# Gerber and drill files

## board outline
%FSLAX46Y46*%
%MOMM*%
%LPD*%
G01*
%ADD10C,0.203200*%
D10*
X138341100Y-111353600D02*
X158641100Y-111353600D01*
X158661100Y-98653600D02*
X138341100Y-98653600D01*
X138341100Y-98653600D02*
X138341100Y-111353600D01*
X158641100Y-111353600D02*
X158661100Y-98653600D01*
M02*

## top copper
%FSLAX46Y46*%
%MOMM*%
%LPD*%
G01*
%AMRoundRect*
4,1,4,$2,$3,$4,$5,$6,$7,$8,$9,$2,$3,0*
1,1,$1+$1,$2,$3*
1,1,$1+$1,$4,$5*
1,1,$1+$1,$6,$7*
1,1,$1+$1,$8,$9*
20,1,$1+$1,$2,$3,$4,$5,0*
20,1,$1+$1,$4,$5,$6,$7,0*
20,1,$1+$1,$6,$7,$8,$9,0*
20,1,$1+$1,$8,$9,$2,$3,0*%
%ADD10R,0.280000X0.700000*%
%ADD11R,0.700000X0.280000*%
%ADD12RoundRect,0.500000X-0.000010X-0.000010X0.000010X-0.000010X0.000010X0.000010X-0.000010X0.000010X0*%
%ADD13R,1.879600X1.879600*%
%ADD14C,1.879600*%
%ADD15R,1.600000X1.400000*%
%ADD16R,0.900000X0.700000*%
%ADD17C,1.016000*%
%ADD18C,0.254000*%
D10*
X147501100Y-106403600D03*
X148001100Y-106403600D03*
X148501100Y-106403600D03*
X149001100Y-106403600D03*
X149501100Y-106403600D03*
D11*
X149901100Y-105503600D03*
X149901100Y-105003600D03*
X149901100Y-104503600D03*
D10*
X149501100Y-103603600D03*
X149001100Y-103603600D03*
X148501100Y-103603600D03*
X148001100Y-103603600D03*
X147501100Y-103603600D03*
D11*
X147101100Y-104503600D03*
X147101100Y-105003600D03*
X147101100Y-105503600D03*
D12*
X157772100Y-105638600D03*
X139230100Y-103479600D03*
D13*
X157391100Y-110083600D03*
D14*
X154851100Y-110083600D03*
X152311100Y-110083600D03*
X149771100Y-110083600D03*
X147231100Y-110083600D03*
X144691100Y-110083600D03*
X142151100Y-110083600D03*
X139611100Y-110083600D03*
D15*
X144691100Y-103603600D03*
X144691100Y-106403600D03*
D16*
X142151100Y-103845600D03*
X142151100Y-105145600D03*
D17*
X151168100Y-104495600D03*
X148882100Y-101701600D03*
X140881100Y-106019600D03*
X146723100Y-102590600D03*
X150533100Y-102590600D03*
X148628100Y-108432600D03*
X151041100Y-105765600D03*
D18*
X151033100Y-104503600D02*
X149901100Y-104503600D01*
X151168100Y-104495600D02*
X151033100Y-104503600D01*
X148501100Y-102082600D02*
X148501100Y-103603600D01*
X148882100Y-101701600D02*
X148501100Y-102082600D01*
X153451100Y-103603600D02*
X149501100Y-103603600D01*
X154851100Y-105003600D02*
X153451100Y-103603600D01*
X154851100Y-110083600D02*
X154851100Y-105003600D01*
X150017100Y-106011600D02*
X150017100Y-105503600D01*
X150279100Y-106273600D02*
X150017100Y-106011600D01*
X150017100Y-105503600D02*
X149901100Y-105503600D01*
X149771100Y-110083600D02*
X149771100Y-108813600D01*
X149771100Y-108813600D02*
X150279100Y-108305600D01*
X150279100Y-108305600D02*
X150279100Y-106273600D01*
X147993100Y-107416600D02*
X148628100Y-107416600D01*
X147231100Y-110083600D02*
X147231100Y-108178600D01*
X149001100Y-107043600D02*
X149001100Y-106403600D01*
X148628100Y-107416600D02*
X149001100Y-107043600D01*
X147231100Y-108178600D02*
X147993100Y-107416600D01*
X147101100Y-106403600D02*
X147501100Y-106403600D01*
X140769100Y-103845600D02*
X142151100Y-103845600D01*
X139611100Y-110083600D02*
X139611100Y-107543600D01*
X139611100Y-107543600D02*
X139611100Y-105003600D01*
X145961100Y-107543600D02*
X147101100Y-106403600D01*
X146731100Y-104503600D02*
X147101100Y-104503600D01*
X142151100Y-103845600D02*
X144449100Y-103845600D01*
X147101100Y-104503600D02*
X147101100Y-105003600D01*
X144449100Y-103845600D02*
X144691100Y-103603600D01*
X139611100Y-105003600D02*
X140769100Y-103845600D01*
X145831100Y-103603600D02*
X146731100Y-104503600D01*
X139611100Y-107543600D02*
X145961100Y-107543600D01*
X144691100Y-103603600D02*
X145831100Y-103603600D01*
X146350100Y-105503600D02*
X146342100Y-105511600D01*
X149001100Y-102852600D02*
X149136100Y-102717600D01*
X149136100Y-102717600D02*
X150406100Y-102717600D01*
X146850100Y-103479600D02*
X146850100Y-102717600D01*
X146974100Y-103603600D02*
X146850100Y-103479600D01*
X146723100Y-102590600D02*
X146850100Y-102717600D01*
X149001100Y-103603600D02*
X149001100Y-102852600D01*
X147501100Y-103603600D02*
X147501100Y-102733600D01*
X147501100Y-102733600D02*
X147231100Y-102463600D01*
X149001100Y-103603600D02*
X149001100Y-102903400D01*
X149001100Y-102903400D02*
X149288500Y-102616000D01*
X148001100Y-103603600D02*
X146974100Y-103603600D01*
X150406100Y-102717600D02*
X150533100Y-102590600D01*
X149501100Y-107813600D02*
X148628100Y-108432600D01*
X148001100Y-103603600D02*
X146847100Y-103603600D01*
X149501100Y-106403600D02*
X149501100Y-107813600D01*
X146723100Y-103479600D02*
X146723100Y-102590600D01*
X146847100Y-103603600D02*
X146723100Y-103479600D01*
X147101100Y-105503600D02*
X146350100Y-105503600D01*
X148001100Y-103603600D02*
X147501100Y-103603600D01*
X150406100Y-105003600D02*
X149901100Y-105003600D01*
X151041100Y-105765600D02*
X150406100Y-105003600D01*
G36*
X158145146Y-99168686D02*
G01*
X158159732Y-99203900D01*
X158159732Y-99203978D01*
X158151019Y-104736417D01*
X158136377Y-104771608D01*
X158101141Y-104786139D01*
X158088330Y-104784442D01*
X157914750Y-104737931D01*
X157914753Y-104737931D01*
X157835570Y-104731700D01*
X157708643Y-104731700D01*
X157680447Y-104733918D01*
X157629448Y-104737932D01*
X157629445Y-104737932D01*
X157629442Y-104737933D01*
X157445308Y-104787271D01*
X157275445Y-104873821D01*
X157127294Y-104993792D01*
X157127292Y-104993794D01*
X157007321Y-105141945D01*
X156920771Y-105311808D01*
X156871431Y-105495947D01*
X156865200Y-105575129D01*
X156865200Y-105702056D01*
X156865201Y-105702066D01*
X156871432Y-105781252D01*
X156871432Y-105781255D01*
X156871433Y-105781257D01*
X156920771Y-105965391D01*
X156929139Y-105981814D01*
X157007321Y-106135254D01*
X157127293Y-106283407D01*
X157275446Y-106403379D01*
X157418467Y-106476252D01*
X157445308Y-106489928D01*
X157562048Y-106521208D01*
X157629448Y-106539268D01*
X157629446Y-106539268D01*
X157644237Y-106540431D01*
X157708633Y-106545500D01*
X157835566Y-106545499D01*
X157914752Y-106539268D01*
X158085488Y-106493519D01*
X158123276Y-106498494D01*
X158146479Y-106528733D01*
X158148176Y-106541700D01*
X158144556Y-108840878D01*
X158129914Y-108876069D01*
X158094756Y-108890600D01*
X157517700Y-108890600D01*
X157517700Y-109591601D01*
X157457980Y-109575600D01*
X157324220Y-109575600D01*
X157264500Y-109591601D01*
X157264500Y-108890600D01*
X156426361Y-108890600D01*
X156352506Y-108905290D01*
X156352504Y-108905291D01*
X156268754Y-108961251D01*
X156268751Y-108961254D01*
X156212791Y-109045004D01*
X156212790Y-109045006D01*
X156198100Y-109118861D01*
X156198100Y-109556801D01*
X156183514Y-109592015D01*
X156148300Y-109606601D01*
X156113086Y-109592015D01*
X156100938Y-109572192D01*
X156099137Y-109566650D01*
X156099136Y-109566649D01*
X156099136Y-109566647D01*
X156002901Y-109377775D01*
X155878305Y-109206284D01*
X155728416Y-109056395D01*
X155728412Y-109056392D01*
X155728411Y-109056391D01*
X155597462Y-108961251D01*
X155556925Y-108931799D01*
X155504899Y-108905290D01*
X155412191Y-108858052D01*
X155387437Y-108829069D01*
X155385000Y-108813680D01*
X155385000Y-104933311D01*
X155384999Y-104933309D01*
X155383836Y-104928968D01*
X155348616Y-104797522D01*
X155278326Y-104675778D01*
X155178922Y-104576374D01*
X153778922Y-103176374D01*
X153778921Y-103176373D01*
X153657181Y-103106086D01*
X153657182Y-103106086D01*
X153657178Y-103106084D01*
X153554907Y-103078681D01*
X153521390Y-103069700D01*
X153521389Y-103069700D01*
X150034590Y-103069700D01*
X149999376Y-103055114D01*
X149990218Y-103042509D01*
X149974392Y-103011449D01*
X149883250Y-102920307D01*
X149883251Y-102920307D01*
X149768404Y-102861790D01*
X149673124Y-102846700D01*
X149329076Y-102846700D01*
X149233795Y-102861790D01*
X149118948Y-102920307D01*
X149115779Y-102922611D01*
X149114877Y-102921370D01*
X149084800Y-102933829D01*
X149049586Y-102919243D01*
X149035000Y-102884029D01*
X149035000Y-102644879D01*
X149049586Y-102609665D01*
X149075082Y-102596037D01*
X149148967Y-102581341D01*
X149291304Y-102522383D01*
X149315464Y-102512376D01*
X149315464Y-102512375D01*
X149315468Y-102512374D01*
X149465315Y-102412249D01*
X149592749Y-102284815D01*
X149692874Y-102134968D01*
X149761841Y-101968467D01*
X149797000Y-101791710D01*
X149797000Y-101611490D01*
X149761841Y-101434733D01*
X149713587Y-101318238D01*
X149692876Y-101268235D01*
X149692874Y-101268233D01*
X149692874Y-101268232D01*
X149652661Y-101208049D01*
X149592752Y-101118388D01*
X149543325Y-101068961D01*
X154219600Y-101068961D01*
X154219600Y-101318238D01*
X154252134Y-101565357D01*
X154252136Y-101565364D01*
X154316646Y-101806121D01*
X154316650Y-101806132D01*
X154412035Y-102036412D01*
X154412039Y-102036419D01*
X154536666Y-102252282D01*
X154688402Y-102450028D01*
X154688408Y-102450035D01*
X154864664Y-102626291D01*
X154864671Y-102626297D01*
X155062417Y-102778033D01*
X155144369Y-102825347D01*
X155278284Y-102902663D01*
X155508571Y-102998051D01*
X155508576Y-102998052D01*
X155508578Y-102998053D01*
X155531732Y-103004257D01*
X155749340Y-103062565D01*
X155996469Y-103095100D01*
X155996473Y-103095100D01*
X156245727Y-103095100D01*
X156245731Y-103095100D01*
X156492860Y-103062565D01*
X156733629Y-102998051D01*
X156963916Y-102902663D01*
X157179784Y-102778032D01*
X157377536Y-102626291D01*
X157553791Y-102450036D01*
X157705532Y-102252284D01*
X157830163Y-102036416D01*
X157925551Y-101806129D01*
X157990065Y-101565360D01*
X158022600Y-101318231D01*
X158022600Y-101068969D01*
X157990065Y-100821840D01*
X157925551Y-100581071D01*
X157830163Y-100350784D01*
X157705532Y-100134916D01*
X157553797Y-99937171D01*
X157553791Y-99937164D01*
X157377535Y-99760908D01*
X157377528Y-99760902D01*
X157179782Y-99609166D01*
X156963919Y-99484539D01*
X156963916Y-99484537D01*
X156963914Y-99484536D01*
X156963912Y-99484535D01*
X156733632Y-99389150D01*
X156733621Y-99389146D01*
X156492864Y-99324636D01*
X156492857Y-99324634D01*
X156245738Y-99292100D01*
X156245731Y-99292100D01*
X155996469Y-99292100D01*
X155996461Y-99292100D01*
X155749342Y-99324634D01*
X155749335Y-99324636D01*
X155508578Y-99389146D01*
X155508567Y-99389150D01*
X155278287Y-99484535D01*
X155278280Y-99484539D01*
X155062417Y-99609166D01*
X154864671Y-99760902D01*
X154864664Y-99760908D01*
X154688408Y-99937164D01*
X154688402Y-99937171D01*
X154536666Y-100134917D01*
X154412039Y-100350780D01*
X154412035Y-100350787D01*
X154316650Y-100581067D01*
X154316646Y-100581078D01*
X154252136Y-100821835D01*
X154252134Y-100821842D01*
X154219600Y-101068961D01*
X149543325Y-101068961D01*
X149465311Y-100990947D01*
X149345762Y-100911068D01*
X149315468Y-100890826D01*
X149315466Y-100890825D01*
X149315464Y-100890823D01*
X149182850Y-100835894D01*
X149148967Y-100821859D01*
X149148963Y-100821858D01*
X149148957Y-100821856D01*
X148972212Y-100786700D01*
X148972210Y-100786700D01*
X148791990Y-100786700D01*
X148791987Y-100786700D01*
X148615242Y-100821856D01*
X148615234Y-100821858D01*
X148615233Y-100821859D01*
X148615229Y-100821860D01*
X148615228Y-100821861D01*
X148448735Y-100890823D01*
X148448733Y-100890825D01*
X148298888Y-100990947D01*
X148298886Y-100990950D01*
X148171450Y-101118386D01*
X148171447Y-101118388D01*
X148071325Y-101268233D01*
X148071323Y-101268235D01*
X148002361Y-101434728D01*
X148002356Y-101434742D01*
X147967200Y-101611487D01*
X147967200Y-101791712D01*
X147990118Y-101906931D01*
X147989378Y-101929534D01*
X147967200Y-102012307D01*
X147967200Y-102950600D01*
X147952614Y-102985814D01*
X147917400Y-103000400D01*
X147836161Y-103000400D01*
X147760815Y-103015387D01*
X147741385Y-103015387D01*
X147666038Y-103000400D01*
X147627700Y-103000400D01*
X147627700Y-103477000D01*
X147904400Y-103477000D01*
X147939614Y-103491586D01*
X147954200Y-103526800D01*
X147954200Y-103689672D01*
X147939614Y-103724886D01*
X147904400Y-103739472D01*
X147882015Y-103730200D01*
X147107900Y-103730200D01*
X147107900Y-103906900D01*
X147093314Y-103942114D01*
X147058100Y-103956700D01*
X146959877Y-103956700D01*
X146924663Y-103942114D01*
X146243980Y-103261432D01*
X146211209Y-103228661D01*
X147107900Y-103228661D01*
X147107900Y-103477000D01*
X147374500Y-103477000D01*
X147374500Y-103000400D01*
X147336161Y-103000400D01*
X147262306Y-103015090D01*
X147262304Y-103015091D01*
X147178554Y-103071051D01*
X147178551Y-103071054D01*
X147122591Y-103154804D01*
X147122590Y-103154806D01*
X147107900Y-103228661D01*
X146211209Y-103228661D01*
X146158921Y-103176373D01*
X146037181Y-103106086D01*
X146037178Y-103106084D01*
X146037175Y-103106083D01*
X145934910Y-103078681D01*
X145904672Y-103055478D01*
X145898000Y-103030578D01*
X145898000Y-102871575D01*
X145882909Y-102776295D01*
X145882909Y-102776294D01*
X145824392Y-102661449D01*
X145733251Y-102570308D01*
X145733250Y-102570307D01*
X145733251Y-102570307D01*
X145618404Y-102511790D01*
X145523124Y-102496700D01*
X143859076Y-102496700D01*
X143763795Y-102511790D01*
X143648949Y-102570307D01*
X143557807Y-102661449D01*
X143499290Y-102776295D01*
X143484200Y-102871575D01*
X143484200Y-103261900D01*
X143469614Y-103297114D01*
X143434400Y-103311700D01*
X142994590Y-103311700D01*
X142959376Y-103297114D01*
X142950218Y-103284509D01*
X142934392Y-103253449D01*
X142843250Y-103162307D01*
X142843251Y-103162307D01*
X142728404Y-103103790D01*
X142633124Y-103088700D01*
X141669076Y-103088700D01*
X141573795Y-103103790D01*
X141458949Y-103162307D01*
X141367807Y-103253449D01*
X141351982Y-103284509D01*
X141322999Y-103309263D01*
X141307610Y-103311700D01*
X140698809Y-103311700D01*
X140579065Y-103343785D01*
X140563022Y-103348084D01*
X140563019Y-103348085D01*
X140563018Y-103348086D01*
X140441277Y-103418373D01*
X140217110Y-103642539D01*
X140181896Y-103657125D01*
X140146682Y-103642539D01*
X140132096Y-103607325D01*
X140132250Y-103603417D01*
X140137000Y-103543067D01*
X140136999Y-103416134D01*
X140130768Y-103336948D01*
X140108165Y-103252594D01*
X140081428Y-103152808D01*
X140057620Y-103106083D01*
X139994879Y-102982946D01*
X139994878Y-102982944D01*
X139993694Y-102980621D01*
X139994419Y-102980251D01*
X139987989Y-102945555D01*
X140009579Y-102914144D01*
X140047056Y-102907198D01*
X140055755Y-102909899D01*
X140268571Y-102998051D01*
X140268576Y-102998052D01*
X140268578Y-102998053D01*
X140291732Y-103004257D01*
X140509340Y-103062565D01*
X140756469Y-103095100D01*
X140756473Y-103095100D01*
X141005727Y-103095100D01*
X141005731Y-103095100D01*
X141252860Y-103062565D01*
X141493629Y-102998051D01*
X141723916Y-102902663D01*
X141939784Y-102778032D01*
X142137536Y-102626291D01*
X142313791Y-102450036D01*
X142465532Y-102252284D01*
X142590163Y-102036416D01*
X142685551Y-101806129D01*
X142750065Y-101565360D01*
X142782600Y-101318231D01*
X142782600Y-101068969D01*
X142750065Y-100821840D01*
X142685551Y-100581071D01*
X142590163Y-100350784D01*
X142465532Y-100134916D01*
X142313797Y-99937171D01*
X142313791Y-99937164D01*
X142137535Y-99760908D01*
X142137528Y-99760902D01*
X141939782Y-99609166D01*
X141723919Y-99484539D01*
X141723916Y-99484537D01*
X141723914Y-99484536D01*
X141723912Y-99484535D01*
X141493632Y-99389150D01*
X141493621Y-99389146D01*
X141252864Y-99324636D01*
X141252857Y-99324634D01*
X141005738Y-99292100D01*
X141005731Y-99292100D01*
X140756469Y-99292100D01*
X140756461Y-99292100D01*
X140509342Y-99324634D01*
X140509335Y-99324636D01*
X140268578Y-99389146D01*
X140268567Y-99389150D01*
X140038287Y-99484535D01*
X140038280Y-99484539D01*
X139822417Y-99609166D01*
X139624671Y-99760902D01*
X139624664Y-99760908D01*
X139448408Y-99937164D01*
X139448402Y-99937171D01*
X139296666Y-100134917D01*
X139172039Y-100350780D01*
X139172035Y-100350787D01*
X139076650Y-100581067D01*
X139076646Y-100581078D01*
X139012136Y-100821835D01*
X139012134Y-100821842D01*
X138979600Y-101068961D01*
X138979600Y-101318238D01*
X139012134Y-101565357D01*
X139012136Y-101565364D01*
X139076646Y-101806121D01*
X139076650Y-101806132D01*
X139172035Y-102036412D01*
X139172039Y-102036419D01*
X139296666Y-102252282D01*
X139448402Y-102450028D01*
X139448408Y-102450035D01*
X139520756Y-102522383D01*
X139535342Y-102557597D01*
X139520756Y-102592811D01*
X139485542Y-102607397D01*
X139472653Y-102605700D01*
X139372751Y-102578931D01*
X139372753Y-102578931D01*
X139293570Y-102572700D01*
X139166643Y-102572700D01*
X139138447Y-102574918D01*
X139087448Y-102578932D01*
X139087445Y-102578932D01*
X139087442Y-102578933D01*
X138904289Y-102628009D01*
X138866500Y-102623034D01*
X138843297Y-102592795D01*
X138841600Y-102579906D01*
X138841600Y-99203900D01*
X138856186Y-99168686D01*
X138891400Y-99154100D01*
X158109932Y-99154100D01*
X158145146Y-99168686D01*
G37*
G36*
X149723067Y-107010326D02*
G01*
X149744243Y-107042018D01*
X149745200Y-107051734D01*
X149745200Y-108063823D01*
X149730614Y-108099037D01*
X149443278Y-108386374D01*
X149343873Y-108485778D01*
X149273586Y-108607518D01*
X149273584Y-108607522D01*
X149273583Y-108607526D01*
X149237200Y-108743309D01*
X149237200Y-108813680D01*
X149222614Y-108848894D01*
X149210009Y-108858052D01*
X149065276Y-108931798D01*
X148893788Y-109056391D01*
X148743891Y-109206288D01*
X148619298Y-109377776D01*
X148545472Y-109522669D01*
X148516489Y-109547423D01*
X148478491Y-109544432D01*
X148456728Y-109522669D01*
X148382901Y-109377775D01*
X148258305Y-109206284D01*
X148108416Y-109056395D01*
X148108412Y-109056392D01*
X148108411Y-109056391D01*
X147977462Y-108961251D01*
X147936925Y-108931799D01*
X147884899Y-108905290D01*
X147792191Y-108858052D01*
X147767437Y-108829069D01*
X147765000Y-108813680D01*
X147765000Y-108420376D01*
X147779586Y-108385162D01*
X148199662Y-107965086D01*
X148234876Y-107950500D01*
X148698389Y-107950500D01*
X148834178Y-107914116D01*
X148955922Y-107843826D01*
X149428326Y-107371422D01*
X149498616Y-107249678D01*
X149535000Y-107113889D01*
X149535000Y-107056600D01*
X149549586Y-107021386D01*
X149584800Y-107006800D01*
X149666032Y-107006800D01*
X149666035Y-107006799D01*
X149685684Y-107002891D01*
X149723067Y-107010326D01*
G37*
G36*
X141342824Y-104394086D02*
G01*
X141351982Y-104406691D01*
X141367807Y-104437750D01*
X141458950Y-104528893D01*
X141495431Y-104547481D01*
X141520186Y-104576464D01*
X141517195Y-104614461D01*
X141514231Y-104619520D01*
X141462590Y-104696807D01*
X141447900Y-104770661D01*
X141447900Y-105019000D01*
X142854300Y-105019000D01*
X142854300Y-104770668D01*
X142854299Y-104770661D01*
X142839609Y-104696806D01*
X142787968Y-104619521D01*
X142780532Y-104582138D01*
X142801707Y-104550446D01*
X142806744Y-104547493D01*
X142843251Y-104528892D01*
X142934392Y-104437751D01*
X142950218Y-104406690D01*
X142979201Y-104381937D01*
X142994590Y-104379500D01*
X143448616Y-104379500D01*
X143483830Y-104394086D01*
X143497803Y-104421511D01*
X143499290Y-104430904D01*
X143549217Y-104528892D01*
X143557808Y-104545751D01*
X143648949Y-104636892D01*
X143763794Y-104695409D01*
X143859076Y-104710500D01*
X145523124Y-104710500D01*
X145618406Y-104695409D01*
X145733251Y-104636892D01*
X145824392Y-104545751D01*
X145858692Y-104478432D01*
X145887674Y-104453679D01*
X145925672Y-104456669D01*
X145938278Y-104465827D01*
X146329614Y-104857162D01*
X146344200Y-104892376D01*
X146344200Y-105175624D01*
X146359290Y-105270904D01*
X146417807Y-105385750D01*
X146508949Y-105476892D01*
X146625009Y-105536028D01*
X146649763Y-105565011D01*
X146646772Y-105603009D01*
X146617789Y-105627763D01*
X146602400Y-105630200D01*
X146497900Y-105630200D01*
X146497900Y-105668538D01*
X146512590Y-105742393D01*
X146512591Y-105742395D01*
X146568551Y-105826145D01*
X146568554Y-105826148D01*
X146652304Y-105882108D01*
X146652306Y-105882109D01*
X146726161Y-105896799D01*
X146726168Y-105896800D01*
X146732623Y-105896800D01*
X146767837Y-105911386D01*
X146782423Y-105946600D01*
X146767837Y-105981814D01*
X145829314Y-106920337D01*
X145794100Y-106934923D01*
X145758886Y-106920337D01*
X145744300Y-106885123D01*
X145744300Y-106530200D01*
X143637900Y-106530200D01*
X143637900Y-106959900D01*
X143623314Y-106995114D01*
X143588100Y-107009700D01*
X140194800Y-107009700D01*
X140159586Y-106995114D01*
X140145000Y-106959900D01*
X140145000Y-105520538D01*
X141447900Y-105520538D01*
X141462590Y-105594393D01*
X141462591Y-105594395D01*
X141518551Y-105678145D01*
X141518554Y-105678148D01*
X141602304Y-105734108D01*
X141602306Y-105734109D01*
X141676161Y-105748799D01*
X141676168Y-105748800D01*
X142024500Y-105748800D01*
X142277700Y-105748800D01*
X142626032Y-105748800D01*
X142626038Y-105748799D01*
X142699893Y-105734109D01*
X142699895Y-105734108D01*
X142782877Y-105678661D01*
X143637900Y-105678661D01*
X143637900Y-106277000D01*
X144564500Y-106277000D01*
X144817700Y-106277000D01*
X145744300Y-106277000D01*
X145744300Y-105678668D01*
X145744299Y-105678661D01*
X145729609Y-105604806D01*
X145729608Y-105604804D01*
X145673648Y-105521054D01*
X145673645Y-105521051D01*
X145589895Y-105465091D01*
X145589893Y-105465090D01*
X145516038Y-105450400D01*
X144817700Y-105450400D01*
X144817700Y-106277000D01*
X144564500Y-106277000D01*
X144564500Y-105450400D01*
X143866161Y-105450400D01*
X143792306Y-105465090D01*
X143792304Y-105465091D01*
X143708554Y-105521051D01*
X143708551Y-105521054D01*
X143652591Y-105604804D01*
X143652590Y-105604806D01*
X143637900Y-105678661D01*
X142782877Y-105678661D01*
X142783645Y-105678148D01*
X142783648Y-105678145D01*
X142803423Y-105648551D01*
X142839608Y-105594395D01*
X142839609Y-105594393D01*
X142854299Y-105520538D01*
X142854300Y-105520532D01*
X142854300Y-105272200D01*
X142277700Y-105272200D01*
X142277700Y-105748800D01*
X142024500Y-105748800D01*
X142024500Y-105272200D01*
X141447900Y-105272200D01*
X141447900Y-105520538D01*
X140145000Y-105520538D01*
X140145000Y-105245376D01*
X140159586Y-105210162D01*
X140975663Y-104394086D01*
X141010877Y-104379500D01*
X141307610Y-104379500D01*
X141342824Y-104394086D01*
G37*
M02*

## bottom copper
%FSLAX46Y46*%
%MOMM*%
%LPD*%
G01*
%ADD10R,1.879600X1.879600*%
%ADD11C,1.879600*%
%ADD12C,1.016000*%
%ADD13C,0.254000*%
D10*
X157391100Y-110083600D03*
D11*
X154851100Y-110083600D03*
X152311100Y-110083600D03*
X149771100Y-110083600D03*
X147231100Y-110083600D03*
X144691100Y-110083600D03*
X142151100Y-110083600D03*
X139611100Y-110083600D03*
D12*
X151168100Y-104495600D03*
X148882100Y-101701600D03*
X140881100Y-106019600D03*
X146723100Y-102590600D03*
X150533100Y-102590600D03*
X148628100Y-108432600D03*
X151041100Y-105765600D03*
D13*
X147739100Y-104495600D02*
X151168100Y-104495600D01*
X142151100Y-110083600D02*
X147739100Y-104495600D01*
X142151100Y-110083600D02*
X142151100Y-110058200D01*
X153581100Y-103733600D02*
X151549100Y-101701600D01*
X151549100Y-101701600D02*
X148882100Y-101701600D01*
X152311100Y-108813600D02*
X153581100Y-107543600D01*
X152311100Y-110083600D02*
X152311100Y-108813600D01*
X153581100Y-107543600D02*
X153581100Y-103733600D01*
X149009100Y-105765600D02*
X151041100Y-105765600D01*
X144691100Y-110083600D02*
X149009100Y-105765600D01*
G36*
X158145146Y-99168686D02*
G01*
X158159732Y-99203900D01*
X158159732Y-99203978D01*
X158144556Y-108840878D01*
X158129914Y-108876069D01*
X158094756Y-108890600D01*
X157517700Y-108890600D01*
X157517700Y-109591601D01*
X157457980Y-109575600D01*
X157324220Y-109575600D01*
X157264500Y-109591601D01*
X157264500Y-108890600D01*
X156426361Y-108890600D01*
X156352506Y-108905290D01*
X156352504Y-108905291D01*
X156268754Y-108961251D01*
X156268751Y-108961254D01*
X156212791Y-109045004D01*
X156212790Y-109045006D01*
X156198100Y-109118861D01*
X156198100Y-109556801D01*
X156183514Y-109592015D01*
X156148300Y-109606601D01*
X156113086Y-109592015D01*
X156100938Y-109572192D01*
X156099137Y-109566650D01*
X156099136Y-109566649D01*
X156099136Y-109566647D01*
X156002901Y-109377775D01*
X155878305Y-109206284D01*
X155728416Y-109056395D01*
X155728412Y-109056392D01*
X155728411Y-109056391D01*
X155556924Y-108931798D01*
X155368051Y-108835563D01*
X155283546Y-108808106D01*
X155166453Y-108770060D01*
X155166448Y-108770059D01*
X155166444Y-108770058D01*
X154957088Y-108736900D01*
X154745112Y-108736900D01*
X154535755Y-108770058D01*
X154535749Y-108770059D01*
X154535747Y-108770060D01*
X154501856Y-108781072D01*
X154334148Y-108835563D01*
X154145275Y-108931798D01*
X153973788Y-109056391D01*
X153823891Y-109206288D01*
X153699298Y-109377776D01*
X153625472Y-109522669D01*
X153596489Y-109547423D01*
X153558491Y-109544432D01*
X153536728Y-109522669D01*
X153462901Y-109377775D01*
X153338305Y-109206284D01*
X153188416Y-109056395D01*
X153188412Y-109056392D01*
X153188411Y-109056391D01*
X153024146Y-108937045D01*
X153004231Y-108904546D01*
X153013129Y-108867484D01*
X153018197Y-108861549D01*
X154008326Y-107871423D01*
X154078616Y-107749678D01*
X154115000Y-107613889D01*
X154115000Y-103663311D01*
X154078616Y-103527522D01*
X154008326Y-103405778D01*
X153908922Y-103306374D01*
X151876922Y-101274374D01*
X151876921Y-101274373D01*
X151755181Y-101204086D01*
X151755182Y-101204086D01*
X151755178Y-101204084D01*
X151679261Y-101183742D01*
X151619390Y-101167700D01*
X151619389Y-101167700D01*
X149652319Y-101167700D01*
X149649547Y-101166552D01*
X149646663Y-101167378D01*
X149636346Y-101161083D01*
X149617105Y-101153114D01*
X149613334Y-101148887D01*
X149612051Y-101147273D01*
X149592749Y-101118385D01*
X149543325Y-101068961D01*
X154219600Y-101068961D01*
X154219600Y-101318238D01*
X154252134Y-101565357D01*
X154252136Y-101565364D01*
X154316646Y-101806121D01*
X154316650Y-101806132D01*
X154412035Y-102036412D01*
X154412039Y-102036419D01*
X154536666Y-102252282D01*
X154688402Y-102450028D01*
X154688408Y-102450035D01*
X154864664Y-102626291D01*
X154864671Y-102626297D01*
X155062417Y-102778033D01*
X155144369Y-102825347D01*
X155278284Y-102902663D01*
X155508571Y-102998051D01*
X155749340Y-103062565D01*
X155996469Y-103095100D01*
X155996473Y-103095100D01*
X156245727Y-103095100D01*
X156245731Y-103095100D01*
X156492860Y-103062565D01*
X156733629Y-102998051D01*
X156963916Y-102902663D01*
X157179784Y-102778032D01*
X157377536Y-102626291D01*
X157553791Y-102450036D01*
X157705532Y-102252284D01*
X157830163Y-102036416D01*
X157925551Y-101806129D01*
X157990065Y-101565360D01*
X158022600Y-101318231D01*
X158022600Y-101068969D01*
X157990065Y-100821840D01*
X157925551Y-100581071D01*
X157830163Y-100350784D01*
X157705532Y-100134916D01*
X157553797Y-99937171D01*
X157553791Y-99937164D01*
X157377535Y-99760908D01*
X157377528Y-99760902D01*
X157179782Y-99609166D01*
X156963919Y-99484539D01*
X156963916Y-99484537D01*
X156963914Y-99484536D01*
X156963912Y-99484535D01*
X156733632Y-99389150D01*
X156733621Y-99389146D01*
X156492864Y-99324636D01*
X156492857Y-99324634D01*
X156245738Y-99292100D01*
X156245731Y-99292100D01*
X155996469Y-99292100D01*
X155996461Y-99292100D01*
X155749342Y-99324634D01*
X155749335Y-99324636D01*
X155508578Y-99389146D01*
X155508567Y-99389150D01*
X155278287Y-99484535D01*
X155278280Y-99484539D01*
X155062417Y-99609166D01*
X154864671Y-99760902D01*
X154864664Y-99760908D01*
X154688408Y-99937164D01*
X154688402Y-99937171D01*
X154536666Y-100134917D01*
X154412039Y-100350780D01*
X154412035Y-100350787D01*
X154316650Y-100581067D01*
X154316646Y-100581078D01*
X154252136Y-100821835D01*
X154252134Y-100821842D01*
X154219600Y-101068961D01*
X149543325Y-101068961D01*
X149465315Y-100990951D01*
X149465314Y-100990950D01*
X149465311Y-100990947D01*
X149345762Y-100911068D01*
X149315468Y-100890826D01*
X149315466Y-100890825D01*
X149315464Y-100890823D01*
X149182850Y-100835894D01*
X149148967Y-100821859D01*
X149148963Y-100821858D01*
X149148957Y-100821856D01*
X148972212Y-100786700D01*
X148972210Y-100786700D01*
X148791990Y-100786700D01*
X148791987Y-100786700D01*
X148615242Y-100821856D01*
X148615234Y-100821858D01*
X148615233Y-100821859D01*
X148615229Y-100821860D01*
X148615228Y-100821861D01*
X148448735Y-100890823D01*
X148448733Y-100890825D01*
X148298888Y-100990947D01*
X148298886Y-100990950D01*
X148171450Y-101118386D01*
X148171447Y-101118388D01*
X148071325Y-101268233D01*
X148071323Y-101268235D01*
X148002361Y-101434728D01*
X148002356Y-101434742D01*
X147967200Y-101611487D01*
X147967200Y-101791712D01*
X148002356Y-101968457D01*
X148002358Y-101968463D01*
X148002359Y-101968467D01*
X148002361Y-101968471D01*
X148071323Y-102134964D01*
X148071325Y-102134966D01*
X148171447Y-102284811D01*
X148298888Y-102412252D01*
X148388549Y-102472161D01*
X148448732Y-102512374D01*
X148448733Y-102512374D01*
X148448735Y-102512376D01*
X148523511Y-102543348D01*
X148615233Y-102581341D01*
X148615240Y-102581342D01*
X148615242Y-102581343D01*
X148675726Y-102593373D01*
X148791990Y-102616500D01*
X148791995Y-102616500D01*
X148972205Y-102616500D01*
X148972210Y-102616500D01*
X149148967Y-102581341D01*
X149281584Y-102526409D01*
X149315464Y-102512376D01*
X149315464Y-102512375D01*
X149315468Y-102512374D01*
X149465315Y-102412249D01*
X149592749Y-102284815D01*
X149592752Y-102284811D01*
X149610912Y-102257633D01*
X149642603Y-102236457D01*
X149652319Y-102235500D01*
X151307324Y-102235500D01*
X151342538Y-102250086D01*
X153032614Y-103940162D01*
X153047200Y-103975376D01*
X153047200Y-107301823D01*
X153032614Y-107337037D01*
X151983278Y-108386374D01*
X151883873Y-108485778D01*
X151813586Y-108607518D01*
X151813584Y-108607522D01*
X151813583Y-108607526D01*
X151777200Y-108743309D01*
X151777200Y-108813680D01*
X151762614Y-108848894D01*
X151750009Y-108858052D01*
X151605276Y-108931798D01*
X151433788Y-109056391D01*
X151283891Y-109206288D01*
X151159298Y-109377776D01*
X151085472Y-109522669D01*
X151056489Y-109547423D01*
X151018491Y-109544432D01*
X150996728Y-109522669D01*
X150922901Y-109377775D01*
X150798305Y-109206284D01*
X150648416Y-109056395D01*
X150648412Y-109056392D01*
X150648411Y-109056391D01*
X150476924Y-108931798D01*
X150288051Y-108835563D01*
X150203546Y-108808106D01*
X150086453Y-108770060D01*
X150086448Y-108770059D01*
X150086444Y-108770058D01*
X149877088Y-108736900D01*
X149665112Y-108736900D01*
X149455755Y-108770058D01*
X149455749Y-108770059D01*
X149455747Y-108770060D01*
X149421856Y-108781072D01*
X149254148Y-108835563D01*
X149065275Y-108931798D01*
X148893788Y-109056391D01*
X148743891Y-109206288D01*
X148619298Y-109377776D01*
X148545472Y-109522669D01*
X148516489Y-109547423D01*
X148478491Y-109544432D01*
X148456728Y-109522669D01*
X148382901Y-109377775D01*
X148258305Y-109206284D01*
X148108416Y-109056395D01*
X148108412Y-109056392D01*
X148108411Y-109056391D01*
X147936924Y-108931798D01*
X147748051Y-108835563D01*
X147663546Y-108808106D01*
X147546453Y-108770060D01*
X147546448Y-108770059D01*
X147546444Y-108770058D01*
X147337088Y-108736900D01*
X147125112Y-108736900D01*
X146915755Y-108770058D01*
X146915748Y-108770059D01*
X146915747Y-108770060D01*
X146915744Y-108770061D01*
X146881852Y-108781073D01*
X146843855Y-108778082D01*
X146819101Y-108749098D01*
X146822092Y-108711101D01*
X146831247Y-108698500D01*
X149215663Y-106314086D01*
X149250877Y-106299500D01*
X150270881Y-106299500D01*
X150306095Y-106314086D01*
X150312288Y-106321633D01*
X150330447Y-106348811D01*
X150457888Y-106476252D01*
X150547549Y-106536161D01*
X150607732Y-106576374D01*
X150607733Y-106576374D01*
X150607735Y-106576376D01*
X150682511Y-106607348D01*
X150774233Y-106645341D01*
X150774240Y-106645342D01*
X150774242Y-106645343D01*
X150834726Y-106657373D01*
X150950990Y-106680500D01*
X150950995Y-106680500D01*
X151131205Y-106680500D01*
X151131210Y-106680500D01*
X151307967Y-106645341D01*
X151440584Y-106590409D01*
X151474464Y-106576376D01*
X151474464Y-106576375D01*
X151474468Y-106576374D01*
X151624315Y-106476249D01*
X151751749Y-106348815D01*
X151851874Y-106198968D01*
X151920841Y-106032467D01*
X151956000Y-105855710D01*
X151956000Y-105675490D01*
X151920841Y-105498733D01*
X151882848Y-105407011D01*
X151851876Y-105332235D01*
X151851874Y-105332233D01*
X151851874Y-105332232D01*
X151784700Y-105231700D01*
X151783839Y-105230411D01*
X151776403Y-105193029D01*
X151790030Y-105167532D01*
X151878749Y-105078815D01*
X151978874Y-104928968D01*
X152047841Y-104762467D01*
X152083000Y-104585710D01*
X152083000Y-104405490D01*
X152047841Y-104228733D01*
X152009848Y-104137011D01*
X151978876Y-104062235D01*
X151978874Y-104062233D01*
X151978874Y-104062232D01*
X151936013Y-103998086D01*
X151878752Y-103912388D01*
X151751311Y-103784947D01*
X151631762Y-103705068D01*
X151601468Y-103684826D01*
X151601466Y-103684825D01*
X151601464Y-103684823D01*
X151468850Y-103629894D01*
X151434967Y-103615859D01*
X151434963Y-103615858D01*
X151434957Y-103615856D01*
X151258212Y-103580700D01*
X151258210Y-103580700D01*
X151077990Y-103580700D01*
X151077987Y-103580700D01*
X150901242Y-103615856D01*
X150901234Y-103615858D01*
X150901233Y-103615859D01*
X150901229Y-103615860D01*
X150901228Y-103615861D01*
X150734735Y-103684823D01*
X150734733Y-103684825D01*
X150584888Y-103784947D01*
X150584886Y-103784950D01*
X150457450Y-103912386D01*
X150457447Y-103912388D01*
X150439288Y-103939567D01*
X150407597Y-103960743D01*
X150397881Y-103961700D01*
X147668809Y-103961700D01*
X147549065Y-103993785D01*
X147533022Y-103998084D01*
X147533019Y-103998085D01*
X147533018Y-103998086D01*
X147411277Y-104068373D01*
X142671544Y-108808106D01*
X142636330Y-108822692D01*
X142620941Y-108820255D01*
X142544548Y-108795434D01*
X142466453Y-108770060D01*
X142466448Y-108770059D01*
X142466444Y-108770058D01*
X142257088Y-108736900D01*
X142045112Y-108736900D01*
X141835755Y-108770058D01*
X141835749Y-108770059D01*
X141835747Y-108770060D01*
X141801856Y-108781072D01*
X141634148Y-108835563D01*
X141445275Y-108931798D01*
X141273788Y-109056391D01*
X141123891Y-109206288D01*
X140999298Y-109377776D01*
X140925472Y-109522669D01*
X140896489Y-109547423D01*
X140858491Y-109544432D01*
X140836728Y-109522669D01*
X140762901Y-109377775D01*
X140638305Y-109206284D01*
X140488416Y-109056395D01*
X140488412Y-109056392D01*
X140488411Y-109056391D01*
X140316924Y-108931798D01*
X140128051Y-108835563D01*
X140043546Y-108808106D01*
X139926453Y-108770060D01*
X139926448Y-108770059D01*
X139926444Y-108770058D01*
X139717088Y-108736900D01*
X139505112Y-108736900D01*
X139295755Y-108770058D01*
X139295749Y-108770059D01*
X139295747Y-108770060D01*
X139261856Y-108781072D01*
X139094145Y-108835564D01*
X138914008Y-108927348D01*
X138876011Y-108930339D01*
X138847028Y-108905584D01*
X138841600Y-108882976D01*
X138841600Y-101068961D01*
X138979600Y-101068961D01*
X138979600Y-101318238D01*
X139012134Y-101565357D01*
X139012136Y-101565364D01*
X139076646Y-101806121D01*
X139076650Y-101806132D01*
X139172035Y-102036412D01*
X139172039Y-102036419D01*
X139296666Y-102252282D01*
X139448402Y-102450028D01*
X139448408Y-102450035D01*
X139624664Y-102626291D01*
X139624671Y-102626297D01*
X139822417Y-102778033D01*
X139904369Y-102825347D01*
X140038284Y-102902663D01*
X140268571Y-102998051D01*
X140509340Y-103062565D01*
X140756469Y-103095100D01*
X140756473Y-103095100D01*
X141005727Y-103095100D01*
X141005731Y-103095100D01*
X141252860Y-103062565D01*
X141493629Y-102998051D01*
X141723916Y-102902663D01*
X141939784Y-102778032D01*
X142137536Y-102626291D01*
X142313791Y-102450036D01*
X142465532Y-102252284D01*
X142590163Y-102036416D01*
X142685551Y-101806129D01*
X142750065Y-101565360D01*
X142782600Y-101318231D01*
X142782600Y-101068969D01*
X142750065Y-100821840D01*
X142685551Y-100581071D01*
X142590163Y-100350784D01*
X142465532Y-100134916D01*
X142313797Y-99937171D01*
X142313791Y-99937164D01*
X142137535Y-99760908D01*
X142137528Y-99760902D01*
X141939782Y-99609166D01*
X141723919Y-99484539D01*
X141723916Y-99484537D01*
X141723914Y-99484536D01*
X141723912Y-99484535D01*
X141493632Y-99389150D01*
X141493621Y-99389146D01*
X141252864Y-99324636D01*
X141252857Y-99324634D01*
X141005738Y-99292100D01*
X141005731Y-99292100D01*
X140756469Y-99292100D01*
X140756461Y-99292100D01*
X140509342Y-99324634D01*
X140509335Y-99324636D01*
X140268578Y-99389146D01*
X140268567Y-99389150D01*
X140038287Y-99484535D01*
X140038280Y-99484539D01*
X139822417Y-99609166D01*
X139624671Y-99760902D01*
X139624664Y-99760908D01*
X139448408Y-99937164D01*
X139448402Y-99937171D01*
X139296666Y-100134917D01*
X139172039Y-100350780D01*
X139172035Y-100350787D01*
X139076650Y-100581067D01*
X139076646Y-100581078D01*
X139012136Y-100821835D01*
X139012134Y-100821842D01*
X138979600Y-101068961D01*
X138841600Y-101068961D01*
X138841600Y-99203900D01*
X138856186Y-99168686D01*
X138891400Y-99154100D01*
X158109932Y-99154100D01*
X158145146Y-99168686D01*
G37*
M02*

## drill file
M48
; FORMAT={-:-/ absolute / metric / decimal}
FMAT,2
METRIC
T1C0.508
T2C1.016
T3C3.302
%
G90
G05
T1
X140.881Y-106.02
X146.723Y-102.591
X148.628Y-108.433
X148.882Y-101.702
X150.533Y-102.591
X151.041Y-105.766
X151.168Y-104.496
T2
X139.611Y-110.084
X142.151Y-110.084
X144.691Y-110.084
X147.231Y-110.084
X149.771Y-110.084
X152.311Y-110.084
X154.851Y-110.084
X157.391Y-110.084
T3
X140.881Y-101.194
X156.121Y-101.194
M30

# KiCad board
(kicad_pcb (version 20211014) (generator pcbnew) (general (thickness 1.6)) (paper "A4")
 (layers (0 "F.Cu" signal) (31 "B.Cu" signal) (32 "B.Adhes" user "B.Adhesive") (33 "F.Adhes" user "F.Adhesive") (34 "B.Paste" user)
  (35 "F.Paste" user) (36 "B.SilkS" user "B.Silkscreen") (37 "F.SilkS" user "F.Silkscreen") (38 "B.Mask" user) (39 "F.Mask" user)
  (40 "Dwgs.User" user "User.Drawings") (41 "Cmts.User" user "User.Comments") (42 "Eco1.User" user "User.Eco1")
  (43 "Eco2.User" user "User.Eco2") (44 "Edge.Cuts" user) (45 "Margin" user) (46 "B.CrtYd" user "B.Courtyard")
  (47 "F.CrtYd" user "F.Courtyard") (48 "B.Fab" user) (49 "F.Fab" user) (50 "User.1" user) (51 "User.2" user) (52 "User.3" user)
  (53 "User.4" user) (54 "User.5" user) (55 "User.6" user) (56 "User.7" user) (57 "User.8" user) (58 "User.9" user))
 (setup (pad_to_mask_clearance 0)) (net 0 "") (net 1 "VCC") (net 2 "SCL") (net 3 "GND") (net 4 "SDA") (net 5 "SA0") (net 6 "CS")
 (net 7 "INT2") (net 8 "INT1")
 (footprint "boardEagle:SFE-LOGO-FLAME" (layer "F.Cu") (at 143.6751 102.0826)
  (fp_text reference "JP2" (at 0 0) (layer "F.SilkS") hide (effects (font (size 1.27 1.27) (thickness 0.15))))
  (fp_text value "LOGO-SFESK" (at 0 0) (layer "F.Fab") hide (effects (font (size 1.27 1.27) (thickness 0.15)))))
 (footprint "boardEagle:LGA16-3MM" (layer "F.Cu") (at 148.5011 105.0036 90)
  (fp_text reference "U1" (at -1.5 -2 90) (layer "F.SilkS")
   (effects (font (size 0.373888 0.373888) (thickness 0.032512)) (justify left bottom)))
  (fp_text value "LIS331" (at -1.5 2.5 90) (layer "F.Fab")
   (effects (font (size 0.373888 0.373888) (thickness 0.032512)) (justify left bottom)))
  (pad "1" smd rect (at -1.4 -1 270) (size 0.7 0.28) (layers "F.Cu" "F.Paste" "F.Mask") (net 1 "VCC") (solder_mask_margin 0.1016))
  (pad "2" smd rect (at -1.4 -0.5 90) (size 0.7 0.28) (layers "F.Cu" "F.Paste" "F.Mask") (solder_mask_margin 0.1016))
  (pad "3" smd rect (at -1.4 0 90) (size 0.7 0.28) (layers "F.Cu" "F.Paste" "F.Mask") (solder_mask_margin 0.1016))
  (pad "4" smd rect (at -1.4 0.5 90) (size 0.7 0.28) (layers "F.Cu" "F.Paste" "F.Mask") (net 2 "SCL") (solder_mask_margin 0.1016))
  (pad "5" smd rect (at -1.4 1 270) (size 0.7 0.28) (layers "F.Cu" "F.Paste" "F.Mask") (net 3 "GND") (solder_mask_margin 0.1016))
  (pad "6" smd rect (at -0.5 1.4 180) (size 0.7 0.28) (layers "F.Cu" "F.Paste" "F.Mask") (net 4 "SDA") (solder_mask_margin 0.1016))
  (pad "7" smd rect (at 0 1.4 180) (size 0.7 0.28) (layers "F.Cu" "F.Paste" "F.Mask") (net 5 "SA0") (solder_mask_margin 0.1016))
  (pad "8" smd rect (at 0.5 1.4 180) (size 0.7 0.28) (layers "F.Cu" "F.Paste" "F.Mask") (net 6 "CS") (solder_mask_margin 0.1016))
  (pad "9" smd rect (at 1.4 1 270) (size 0.7 0.28) (layers "F.Cu" "F.Paste" "F.Mask") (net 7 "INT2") (solder_mask_margin 0.1016))
  (pad "10" smd rect (at 1.4 0.5 270) (size 0.7 0.28) (layers "F.Cu" "F.Paste" "F.Mask") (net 3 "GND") (solder_mask_margin 0.1016))
  (pad "11" smd rect (at 1.4 0 270) (size 0.7 0.28) (layers "F.Cu" "F.Paste" "F.Mask") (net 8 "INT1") (solder_mask_margin 0.1016))
  (pad "12" smd rect (at 1.4 -0.5 270) (size 0.7 0.28) (layers "F.Cu" "F.Paste" "F.Mask") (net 3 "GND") (solder_mask_margin 0.1016))
  (pad "13" smd rect (at 1.4 -1 270) (size 0.7 0.28) (layers "F.Cu" "F.Paste" "F.Mask") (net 3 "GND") (solder_mask_margin 0.1016))
  (pad "14" smd rect (at 0.5 -1.4) (size 0.7 0.28) (layers "F.Cu" "F.Paste" "F.Mask") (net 1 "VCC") (solder_mask_margin 0.1016))
  (pad "15" smd rect (at 0 -1.4) (size 0.7 0.28) (layers "F.Cu" "F.Paste" "F.Mask") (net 1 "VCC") (solder_mask_margin 0.1016))
  (pad "16" smd rect (at -0.5 -1.4) (size 0.7 0.28) (layers "F.Cu" "F.Paste" "F.Mask") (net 3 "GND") (solder_mask_margin 0.1016)))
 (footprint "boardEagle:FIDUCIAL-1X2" (layer "F.Cu") (at 157.7721 105.6386)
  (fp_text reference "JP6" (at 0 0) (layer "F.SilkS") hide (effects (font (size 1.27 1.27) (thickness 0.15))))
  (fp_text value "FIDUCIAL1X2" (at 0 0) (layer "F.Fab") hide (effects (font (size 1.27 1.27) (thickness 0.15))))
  (pad "1" smd roundrect (at 0 0) (size 1 1) (layers "F.Cu" "F.Mask") (roundrect_rratio 0.5) (solder_mask_margin 0.1016)))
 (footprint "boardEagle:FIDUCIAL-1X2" (layer "F.Cu") (at 139.2301 103.4796)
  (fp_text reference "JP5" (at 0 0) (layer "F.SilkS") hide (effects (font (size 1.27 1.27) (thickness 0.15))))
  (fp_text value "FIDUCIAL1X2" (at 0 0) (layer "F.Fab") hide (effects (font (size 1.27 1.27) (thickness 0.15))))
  (pad "1" smd roundrect (at 0 0) (size 1 1) (layers "F.Cu" "F.Mask") (roundrect_rratio 0.5) (solder_mask_margin 0.1016)))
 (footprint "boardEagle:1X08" (layer "F.Cu") (at 157.3911 110.0836 180)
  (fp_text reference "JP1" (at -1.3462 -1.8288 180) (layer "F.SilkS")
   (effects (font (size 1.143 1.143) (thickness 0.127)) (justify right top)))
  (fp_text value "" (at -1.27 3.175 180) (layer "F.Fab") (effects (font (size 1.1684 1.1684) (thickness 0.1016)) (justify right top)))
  (pad "1" thru_hole rect (at 0 0 270) (size 1.8796 1.8796) (drill 1.016) (layers *.Cu *.Mask) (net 3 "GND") (solder_mask_margin 0.1016))
  (pad "2" thru_hole circle (at 2.54 0 270) (size 1.8796 1.8796) (drill 1.016) (layers *.Cu *.Mask) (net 7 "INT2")
   (solder_mask_margin 0.1016))
  (pad "3" thru_hole circle (at 5.08 0 270) (size 1.8796 1.8796) (drill 1.016) (layers *.Cu *.Mask) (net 8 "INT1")
   (solder_mask_margin 0.1016))
  (pad "4" thru_hole circle (at 7.62 0 270) (size 1.8796 1.8796) (drill 1.016) (layers *.Cu *.Mask) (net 4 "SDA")
   (solder_mask_margin 0.1016))
  (pad "5" thru_hole circle (at 10.16 0 270) (size 1.8796 1.8796) (drill 1.016) (layers *.Cu *.Mask) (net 2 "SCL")
   (solder_mask_margin 0.1016))
  (pad "6" thru_hole circle (at 12.7 0 270) (size 1.8796 1.8796) (drill 1.016) (layers *.Cu *.Mask) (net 5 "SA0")
   (solder_mask_margin 0.1016))
  (pad "7" thru_hole circle (at 15.24 0 270) (size 1.8796 1.8796) (drill 1.016) (layers *.Cu *.Mask) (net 6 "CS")
   (solder_mask_margin 0.1016))
  (pad "8" thru_hole circle (at 17.78 0 270) (size 1.8796 1.8796) (drill 1.016) (layers *.Cu *.Mask) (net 1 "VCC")
   (solder_mask_margin 0.1016)))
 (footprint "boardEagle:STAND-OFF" (layer "F.Cu") (at 140.8811 101.1936)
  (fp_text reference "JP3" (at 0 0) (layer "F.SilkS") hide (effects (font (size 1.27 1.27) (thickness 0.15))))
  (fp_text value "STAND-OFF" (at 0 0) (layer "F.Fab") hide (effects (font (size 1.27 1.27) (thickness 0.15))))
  (pad "" np_thru_hole circle (at 0 0) (size 3.302 3.302) (drill 3.302) (layers *.Cu *.Mask)))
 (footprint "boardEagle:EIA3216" (layer "F.Cu") (at 144.6911 105.0036 90)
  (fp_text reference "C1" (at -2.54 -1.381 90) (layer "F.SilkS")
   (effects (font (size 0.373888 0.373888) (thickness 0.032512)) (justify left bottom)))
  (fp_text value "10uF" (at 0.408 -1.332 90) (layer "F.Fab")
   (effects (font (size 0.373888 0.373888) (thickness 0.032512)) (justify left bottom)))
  (pad "A" smd rect (at 1.4 0 180) (size 1.6 1.4) (layers "F.Cu" "F.Paste" "F.Mask") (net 1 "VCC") (solder_mask_margin 0.1016))
  (pad "C" smd rect (at -1.4 0 180) (size 1.6 1.4) (layers "F.Cu" "F.Paste" "F.Mask") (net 3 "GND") (solder_mask_margin 0.1016)))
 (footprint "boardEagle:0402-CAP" (layer "F.Cu") (at 142.1511 104.4956 -90)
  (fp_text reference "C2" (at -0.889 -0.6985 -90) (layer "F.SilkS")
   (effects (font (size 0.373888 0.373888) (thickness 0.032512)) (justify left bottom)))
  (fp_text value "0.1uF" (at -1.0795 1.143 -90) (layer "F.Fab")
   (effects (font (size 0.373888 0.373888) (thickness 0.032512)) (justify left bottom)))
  (pad "1" smd rect (at -0.65 0 270) (size 0.7 0.9) (layers "F.Cu" "F.Paste" "F.Mask") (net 1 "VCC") (solder_mask_margin 0.1016))
  (pad "2" smd rect (at 0.65 0 270) (size 0.7 0.9) (layers "F.Cu" "F.Paste" "F.Mask") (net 3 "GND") (solder_mask_margin 0.1016)))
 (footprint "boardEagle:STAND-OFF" (layer "F.Cu") (at 156.1211 101.1936)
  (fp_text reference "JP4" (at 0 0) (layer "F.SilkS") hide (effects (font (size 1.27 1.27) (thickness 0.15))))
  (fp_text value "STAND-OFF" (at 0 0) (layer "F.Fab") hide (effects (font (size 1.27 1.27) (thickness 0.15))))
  (pad "" np_thru_hole circle (at 0 0) (size 3.302 3.302) (drill 3.302) (layers *.Cu *.Mask)))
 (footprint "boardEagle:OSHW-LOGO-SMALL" (layer "B.Cu") (at 145.0721 101.0666 -90)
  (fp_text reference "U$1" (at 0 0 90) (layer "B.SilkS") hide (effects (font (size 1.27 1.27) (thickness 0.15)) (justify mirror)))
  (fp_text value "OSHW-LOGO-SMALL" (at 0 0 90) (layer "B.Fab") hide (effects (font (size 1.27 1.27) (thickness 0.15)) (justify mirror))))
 (gr_line (start 138.3411 111.3536) (end 158.6411 111.3536) (layer "Edge.Cuts") (width 0.2032))
 (gr_line (start 158.6611 98.6536) (end 138.3411 98.6536) (layer "Edge.Cuts") (width 0.2032))
 (gr_line (start 138.3411 98.6536) (end 138.3411 111.3536) (layer "Edge.Cuts") (width 0.2032))
 (gr_line (start 158.6411 111.3536) (end 158.6611 98.6536) (layer "Edge.Cuts") (width 0.2032))
 (segment (start 151.0331 104.5036) (end 149.9011 104.5036) (width 0.254) (layer "F.Cu") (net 6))
 (segment (start 151.1681 104.4956) (end 151.0331 104.5036) (width 0.254) (layer "F.Cu") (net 6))
 (via (at 151.1681 104.4956) (size 1.016) (drill 0.508) (layers "F.Cu" "B.Cu") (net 6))
 (segment (start 147.7391 104.4956) (end 151.1681 104.4956) (width 0.254) (layer "B.Cu") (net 6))
 (segment (start 142.1511 110.0836) (end 147.7391 104.4956) (width 0.254) (layer "B.Cu") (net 6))
 (segment (start 142.1511 110.0836) (end 142.1511 110.0582) (width 0.254) (layer "B.Cu") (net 6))
 (segment (start 148.5011 102.0826) (end 148.5011 103.6036) (width 0.254) (layer "F.Cu") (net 8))
 (segment (start 148.8821 101.7016) (end 148.5011 102.0826) (width 0.254) (layer "F.Cu") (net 8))
 (via (at 148.8821 101.7016) (size 1.016) (drill 0.508) (layers "F.Cu" "B.Cu") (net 8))
 (segment (start 153.5811 103.7336) (end 151.5491 101.7016) (width 0.254) (layer "B.Cu") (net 8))
 (segment (start 151.5491 101.7016) (end 148.8821 101.7016) (width 0.254) (layer "B.Cu") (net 8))
 (segment (start 152.3111 108.8136) (end 153.5811 107.5436) (width 0.254) (layer "B.Cu") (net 8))
 (segment (start 152.3111 110.0836) (end 152.3111 108.8136) (width 0.254) (layer "B.Cu") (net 8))
 (segment (start 153.5811 107.5436) (end 153.5811 103.7336) (width 0.254) (layer "B.Cu") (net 8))
 (segment (start 153.4511 103.6036) (end 149.5011 103.6036) (width 0.254) (layer "F.Cu") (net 7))
 (segment (start 154.8511 105.0036) (end 153.4511 103.6036) (width 0.254) (layer "F.Cu") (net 7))
 (segment (start 154.8511 110.0836) (end 154.8511 105.0036) (width 0.254) (layer "F.Cu") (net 7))
 (segment (start 150.0171 106.0116) (end 150.0171 105.5036) (width 0.254) (layer "F.Cu") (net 4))
 (segment (start 150.2791 106.2736) (end 150.0171 106.0116) (width 0.254) (layer "F.Cu") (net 4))
 (segment (start 150.0171 105.5036) (end 149.9011 105.5036) (width 0.254) (layer "F.Cu") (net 4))
 (segment (start 149.7711 110.0836) (end 149.7711 108.8136) (width 0.254) (layer "F.Cu") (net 4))
 (segment (start 149.7711 108.8136) (end 150.2791 108.3056) (width 0.254) (layer "F.Cu") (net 4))
 (segment (start 150.2791 108.3056) (end 150.2791 106.2736) (width 0.254) (layer "F.Cu") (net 4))
 (segment (start 147.9931 107.4166) (end 148.6281 107.4166) (width 0.254) (layer "F.Cu") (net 2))
 (segment (start 147.2311 110.0836) (end 147.2311 108.1786) (width 0.254) (layer "F.Cu") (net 2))
 (segment (start 149.0011 107.0436) (end 149.0011 106.4036) (width 0.254) (layer "F.Cu") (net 2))
 (segment (start 148.6281 107.4166) (end 149.0011 107.0436) (width 0.254) (layer "F.Cu") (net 2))
 (segment (start 147.2311 108.1786) (end 147.9931 107.4166) (width 0.254) (layer "F.Cu") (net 2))
 (segment (start 147.1011 106.4036) (end 147.5011 106.4036) (width 0.254) (layer "F.Cu") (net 1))
 (segment (start 140.7691 103.8456) (end 142.1511 103.8456) (width 0.254) (layer "F.Cu") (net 1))
 (segment (start 139.6111 110.0836) (end 139.6111 107.5436) (width 0.254) (layer "F.Cu") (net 1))
 (segment (start 139.6111 107.5436) (end 139.6111 105.0036) (width 0.254) (layer "F.Cu") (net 1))
 (segment (start 145.9611 107.5436) (end 147.1011 106.4036) (width 0.254) (layer "F.Cu") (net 1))
 (segment (start 146.7311 104.5036) (end 147.1011 104.5036) (width 0.254) (layer "F.Cu") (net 1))
 (segment (start 142.1511 103.8456) (end 144.4491 103.8456) (width 0.254) (layer "F.Cu") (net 1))
 (segment (start 147.1011 104.5036) (end 147.1011 105.0036) (width 0.254) (layer "F.Cu") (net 1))
 (segment (start 144.4491 103.8456) (end 144.6911 103.6036) (width 0.254) (layer "F.Cu") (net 1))
 (segment (start 139.6111 105.0036) (end 140.7691 103.8456) (width 0.254) (layer "F.Cu") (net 1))
 (segment (start 145.8311 103.6036) (end 146.7311 104.5036) (width 0.254) (layer "F.Cu") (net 1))
 (segment (start 139.6111 107.5436) (end 145.9611 107.5436) (width 0.254) (layer "F.Cu") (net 1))
 (segment (start 144.6911 103.6036) (end 145.8311 103.6036) (width 0.254) (layer "F.Cu") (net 1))
 (segment (start 146.3501 105.5036) (end 146.3421 105.5116) (width 0.254) (layer "F.Cu") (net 3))
 (segment (start 149.0011 102.8526) (end 149.1361 102.7176) (width 0.254) (layer "F.Cu") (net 3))
 (segment (start 149.1361 102.7176) (end 150.4061 102.7176) (width 0.254) (layer "F.Cu") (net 3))
 (segment (start 146.8501 103.4796) (end 146.8501 102.7176) (width 0.254) (layer "F.Cu") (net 3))
 (segment (start 146.9741 103.6036) (end 146.8501 103.4796) (width 0.254) (layer "F.Cu") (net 3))
 (segment (start 146.7231 102.5906) (end 146.8501 102.7176) (width 0.254) (layer "F.Cu") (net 3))
 (segment (start 149.0011 103.6036) (end 149.0011 102.8526) (width 0.254) (layer "F.Cu") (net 3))
 (segment (start 147.5011 103.6036) (end 147.5011 102.7336) (width 0.254) (layer "F.Cu") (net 3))
 (segment (start 147.5011 102.7336) (end 147.2311 102.4636) (width 0.254) (layer "F.Cu") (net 3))
 (segment (start 149.0011 103.6036) (end 149.0011 102.9034) (width 0.254) (layer "F.Cu") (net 3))
 (segment (start 149.0011 102.9034) (end 149.2885 102.616) (width 0.254) (layer "F.Cu") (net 3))
 (segment (start 148.0011 103.6036) (end 146.9741 103.6036) (width 0.254) (layer "F.Cu") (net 3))
 (segment (start 150.4061 102.7176) (end 150.5331 102.5906) (width 0.254) (layer "F.Cu") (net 3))
 (segment (start 149.5011 107.8136) (end 148.6281 108.4326) (width 0.254) (layer "F.Cu") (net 3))
 (segment (start 148.0011 103.6036) (end 146.8471 103.6036) (width 0.254) (layer "F.Cu") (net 3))
 (segment (start 149.5011 106.4036) (end 149.5011 107.8136) (width 0.254) (layer "F.Cu") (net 3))
 (segment (start 146.7231 103.4796) (end 146.7231 102.5906) (width 0.254) (layer "F.Cu") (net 3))
 (segment (start 146.8471 103.6036) (end 146.7231 103.4796) (width 0.254) (layer "F.Cu") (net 3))
 (segment (start 147.1011 105.5036) (end 146.3501 105.5036) (width 0.254) (layer "F.Cu") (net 3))
 (segment (start 148.0011 103.6036) (end 147.5011 103.6036) (width 0.254) (layer "F.Cu") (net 3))
 (via (at 140.8811 106.0196) (size 1.016) (drill 0.508) (layers "F.Cu" "B.Cu") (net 3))
 (via (at 146.7231 102.5906) (size 1.016) (drill 0.508) (layers "F.Cu" "B.Cu") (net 3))
 (via (at 150.5331 102.5906) (size 1.016) (drill 0.508) (layers "F.Cu" "B.Cu") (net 3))
 (via (at 148.6281 108.4326) (size 1.016) (drill 0.508) (layers "F.Cu" "B.Cu") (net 3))
 (segment (start 150.4061 105.0036) (end 149.9011 105.0036) (width 0.254) (layer "F.Cu") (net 5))
 (segment (start 151.0411 105.7656) (end 150.4061 105.0036) (width 0.254) (layer "F.Cu") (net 5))
 (via (at 151.0411 105.7656) (size 1.016) (drill 0.508) (layers "F.Cu" "B.Cu") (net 5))
 (segment (start 149.0091 105.7656) (end 151.0411 105.7656) (width 0.254) (layer "B.Cu") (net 5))
 (segment (start 144.6911 110.0836) (end 149.0091 105.7656) (width 0.254) (layer "B.Cu") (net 5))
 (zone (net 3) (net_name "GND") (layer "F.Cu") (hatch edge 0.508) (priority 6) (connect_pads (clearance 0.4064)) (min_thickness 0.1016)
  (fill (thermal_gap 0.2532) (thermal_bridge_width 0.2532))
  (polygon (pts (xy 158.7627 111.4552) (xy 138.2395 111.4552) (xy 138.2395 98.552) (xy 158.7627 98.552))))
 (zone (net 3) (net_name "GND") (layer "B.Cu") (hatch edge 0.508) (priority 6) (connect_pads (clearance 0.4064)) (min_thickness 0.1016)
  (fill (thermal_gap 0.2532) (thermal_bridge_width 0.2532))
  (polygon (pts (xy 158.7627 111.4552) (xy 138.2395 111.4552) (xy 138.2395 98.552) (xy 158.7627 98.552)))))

